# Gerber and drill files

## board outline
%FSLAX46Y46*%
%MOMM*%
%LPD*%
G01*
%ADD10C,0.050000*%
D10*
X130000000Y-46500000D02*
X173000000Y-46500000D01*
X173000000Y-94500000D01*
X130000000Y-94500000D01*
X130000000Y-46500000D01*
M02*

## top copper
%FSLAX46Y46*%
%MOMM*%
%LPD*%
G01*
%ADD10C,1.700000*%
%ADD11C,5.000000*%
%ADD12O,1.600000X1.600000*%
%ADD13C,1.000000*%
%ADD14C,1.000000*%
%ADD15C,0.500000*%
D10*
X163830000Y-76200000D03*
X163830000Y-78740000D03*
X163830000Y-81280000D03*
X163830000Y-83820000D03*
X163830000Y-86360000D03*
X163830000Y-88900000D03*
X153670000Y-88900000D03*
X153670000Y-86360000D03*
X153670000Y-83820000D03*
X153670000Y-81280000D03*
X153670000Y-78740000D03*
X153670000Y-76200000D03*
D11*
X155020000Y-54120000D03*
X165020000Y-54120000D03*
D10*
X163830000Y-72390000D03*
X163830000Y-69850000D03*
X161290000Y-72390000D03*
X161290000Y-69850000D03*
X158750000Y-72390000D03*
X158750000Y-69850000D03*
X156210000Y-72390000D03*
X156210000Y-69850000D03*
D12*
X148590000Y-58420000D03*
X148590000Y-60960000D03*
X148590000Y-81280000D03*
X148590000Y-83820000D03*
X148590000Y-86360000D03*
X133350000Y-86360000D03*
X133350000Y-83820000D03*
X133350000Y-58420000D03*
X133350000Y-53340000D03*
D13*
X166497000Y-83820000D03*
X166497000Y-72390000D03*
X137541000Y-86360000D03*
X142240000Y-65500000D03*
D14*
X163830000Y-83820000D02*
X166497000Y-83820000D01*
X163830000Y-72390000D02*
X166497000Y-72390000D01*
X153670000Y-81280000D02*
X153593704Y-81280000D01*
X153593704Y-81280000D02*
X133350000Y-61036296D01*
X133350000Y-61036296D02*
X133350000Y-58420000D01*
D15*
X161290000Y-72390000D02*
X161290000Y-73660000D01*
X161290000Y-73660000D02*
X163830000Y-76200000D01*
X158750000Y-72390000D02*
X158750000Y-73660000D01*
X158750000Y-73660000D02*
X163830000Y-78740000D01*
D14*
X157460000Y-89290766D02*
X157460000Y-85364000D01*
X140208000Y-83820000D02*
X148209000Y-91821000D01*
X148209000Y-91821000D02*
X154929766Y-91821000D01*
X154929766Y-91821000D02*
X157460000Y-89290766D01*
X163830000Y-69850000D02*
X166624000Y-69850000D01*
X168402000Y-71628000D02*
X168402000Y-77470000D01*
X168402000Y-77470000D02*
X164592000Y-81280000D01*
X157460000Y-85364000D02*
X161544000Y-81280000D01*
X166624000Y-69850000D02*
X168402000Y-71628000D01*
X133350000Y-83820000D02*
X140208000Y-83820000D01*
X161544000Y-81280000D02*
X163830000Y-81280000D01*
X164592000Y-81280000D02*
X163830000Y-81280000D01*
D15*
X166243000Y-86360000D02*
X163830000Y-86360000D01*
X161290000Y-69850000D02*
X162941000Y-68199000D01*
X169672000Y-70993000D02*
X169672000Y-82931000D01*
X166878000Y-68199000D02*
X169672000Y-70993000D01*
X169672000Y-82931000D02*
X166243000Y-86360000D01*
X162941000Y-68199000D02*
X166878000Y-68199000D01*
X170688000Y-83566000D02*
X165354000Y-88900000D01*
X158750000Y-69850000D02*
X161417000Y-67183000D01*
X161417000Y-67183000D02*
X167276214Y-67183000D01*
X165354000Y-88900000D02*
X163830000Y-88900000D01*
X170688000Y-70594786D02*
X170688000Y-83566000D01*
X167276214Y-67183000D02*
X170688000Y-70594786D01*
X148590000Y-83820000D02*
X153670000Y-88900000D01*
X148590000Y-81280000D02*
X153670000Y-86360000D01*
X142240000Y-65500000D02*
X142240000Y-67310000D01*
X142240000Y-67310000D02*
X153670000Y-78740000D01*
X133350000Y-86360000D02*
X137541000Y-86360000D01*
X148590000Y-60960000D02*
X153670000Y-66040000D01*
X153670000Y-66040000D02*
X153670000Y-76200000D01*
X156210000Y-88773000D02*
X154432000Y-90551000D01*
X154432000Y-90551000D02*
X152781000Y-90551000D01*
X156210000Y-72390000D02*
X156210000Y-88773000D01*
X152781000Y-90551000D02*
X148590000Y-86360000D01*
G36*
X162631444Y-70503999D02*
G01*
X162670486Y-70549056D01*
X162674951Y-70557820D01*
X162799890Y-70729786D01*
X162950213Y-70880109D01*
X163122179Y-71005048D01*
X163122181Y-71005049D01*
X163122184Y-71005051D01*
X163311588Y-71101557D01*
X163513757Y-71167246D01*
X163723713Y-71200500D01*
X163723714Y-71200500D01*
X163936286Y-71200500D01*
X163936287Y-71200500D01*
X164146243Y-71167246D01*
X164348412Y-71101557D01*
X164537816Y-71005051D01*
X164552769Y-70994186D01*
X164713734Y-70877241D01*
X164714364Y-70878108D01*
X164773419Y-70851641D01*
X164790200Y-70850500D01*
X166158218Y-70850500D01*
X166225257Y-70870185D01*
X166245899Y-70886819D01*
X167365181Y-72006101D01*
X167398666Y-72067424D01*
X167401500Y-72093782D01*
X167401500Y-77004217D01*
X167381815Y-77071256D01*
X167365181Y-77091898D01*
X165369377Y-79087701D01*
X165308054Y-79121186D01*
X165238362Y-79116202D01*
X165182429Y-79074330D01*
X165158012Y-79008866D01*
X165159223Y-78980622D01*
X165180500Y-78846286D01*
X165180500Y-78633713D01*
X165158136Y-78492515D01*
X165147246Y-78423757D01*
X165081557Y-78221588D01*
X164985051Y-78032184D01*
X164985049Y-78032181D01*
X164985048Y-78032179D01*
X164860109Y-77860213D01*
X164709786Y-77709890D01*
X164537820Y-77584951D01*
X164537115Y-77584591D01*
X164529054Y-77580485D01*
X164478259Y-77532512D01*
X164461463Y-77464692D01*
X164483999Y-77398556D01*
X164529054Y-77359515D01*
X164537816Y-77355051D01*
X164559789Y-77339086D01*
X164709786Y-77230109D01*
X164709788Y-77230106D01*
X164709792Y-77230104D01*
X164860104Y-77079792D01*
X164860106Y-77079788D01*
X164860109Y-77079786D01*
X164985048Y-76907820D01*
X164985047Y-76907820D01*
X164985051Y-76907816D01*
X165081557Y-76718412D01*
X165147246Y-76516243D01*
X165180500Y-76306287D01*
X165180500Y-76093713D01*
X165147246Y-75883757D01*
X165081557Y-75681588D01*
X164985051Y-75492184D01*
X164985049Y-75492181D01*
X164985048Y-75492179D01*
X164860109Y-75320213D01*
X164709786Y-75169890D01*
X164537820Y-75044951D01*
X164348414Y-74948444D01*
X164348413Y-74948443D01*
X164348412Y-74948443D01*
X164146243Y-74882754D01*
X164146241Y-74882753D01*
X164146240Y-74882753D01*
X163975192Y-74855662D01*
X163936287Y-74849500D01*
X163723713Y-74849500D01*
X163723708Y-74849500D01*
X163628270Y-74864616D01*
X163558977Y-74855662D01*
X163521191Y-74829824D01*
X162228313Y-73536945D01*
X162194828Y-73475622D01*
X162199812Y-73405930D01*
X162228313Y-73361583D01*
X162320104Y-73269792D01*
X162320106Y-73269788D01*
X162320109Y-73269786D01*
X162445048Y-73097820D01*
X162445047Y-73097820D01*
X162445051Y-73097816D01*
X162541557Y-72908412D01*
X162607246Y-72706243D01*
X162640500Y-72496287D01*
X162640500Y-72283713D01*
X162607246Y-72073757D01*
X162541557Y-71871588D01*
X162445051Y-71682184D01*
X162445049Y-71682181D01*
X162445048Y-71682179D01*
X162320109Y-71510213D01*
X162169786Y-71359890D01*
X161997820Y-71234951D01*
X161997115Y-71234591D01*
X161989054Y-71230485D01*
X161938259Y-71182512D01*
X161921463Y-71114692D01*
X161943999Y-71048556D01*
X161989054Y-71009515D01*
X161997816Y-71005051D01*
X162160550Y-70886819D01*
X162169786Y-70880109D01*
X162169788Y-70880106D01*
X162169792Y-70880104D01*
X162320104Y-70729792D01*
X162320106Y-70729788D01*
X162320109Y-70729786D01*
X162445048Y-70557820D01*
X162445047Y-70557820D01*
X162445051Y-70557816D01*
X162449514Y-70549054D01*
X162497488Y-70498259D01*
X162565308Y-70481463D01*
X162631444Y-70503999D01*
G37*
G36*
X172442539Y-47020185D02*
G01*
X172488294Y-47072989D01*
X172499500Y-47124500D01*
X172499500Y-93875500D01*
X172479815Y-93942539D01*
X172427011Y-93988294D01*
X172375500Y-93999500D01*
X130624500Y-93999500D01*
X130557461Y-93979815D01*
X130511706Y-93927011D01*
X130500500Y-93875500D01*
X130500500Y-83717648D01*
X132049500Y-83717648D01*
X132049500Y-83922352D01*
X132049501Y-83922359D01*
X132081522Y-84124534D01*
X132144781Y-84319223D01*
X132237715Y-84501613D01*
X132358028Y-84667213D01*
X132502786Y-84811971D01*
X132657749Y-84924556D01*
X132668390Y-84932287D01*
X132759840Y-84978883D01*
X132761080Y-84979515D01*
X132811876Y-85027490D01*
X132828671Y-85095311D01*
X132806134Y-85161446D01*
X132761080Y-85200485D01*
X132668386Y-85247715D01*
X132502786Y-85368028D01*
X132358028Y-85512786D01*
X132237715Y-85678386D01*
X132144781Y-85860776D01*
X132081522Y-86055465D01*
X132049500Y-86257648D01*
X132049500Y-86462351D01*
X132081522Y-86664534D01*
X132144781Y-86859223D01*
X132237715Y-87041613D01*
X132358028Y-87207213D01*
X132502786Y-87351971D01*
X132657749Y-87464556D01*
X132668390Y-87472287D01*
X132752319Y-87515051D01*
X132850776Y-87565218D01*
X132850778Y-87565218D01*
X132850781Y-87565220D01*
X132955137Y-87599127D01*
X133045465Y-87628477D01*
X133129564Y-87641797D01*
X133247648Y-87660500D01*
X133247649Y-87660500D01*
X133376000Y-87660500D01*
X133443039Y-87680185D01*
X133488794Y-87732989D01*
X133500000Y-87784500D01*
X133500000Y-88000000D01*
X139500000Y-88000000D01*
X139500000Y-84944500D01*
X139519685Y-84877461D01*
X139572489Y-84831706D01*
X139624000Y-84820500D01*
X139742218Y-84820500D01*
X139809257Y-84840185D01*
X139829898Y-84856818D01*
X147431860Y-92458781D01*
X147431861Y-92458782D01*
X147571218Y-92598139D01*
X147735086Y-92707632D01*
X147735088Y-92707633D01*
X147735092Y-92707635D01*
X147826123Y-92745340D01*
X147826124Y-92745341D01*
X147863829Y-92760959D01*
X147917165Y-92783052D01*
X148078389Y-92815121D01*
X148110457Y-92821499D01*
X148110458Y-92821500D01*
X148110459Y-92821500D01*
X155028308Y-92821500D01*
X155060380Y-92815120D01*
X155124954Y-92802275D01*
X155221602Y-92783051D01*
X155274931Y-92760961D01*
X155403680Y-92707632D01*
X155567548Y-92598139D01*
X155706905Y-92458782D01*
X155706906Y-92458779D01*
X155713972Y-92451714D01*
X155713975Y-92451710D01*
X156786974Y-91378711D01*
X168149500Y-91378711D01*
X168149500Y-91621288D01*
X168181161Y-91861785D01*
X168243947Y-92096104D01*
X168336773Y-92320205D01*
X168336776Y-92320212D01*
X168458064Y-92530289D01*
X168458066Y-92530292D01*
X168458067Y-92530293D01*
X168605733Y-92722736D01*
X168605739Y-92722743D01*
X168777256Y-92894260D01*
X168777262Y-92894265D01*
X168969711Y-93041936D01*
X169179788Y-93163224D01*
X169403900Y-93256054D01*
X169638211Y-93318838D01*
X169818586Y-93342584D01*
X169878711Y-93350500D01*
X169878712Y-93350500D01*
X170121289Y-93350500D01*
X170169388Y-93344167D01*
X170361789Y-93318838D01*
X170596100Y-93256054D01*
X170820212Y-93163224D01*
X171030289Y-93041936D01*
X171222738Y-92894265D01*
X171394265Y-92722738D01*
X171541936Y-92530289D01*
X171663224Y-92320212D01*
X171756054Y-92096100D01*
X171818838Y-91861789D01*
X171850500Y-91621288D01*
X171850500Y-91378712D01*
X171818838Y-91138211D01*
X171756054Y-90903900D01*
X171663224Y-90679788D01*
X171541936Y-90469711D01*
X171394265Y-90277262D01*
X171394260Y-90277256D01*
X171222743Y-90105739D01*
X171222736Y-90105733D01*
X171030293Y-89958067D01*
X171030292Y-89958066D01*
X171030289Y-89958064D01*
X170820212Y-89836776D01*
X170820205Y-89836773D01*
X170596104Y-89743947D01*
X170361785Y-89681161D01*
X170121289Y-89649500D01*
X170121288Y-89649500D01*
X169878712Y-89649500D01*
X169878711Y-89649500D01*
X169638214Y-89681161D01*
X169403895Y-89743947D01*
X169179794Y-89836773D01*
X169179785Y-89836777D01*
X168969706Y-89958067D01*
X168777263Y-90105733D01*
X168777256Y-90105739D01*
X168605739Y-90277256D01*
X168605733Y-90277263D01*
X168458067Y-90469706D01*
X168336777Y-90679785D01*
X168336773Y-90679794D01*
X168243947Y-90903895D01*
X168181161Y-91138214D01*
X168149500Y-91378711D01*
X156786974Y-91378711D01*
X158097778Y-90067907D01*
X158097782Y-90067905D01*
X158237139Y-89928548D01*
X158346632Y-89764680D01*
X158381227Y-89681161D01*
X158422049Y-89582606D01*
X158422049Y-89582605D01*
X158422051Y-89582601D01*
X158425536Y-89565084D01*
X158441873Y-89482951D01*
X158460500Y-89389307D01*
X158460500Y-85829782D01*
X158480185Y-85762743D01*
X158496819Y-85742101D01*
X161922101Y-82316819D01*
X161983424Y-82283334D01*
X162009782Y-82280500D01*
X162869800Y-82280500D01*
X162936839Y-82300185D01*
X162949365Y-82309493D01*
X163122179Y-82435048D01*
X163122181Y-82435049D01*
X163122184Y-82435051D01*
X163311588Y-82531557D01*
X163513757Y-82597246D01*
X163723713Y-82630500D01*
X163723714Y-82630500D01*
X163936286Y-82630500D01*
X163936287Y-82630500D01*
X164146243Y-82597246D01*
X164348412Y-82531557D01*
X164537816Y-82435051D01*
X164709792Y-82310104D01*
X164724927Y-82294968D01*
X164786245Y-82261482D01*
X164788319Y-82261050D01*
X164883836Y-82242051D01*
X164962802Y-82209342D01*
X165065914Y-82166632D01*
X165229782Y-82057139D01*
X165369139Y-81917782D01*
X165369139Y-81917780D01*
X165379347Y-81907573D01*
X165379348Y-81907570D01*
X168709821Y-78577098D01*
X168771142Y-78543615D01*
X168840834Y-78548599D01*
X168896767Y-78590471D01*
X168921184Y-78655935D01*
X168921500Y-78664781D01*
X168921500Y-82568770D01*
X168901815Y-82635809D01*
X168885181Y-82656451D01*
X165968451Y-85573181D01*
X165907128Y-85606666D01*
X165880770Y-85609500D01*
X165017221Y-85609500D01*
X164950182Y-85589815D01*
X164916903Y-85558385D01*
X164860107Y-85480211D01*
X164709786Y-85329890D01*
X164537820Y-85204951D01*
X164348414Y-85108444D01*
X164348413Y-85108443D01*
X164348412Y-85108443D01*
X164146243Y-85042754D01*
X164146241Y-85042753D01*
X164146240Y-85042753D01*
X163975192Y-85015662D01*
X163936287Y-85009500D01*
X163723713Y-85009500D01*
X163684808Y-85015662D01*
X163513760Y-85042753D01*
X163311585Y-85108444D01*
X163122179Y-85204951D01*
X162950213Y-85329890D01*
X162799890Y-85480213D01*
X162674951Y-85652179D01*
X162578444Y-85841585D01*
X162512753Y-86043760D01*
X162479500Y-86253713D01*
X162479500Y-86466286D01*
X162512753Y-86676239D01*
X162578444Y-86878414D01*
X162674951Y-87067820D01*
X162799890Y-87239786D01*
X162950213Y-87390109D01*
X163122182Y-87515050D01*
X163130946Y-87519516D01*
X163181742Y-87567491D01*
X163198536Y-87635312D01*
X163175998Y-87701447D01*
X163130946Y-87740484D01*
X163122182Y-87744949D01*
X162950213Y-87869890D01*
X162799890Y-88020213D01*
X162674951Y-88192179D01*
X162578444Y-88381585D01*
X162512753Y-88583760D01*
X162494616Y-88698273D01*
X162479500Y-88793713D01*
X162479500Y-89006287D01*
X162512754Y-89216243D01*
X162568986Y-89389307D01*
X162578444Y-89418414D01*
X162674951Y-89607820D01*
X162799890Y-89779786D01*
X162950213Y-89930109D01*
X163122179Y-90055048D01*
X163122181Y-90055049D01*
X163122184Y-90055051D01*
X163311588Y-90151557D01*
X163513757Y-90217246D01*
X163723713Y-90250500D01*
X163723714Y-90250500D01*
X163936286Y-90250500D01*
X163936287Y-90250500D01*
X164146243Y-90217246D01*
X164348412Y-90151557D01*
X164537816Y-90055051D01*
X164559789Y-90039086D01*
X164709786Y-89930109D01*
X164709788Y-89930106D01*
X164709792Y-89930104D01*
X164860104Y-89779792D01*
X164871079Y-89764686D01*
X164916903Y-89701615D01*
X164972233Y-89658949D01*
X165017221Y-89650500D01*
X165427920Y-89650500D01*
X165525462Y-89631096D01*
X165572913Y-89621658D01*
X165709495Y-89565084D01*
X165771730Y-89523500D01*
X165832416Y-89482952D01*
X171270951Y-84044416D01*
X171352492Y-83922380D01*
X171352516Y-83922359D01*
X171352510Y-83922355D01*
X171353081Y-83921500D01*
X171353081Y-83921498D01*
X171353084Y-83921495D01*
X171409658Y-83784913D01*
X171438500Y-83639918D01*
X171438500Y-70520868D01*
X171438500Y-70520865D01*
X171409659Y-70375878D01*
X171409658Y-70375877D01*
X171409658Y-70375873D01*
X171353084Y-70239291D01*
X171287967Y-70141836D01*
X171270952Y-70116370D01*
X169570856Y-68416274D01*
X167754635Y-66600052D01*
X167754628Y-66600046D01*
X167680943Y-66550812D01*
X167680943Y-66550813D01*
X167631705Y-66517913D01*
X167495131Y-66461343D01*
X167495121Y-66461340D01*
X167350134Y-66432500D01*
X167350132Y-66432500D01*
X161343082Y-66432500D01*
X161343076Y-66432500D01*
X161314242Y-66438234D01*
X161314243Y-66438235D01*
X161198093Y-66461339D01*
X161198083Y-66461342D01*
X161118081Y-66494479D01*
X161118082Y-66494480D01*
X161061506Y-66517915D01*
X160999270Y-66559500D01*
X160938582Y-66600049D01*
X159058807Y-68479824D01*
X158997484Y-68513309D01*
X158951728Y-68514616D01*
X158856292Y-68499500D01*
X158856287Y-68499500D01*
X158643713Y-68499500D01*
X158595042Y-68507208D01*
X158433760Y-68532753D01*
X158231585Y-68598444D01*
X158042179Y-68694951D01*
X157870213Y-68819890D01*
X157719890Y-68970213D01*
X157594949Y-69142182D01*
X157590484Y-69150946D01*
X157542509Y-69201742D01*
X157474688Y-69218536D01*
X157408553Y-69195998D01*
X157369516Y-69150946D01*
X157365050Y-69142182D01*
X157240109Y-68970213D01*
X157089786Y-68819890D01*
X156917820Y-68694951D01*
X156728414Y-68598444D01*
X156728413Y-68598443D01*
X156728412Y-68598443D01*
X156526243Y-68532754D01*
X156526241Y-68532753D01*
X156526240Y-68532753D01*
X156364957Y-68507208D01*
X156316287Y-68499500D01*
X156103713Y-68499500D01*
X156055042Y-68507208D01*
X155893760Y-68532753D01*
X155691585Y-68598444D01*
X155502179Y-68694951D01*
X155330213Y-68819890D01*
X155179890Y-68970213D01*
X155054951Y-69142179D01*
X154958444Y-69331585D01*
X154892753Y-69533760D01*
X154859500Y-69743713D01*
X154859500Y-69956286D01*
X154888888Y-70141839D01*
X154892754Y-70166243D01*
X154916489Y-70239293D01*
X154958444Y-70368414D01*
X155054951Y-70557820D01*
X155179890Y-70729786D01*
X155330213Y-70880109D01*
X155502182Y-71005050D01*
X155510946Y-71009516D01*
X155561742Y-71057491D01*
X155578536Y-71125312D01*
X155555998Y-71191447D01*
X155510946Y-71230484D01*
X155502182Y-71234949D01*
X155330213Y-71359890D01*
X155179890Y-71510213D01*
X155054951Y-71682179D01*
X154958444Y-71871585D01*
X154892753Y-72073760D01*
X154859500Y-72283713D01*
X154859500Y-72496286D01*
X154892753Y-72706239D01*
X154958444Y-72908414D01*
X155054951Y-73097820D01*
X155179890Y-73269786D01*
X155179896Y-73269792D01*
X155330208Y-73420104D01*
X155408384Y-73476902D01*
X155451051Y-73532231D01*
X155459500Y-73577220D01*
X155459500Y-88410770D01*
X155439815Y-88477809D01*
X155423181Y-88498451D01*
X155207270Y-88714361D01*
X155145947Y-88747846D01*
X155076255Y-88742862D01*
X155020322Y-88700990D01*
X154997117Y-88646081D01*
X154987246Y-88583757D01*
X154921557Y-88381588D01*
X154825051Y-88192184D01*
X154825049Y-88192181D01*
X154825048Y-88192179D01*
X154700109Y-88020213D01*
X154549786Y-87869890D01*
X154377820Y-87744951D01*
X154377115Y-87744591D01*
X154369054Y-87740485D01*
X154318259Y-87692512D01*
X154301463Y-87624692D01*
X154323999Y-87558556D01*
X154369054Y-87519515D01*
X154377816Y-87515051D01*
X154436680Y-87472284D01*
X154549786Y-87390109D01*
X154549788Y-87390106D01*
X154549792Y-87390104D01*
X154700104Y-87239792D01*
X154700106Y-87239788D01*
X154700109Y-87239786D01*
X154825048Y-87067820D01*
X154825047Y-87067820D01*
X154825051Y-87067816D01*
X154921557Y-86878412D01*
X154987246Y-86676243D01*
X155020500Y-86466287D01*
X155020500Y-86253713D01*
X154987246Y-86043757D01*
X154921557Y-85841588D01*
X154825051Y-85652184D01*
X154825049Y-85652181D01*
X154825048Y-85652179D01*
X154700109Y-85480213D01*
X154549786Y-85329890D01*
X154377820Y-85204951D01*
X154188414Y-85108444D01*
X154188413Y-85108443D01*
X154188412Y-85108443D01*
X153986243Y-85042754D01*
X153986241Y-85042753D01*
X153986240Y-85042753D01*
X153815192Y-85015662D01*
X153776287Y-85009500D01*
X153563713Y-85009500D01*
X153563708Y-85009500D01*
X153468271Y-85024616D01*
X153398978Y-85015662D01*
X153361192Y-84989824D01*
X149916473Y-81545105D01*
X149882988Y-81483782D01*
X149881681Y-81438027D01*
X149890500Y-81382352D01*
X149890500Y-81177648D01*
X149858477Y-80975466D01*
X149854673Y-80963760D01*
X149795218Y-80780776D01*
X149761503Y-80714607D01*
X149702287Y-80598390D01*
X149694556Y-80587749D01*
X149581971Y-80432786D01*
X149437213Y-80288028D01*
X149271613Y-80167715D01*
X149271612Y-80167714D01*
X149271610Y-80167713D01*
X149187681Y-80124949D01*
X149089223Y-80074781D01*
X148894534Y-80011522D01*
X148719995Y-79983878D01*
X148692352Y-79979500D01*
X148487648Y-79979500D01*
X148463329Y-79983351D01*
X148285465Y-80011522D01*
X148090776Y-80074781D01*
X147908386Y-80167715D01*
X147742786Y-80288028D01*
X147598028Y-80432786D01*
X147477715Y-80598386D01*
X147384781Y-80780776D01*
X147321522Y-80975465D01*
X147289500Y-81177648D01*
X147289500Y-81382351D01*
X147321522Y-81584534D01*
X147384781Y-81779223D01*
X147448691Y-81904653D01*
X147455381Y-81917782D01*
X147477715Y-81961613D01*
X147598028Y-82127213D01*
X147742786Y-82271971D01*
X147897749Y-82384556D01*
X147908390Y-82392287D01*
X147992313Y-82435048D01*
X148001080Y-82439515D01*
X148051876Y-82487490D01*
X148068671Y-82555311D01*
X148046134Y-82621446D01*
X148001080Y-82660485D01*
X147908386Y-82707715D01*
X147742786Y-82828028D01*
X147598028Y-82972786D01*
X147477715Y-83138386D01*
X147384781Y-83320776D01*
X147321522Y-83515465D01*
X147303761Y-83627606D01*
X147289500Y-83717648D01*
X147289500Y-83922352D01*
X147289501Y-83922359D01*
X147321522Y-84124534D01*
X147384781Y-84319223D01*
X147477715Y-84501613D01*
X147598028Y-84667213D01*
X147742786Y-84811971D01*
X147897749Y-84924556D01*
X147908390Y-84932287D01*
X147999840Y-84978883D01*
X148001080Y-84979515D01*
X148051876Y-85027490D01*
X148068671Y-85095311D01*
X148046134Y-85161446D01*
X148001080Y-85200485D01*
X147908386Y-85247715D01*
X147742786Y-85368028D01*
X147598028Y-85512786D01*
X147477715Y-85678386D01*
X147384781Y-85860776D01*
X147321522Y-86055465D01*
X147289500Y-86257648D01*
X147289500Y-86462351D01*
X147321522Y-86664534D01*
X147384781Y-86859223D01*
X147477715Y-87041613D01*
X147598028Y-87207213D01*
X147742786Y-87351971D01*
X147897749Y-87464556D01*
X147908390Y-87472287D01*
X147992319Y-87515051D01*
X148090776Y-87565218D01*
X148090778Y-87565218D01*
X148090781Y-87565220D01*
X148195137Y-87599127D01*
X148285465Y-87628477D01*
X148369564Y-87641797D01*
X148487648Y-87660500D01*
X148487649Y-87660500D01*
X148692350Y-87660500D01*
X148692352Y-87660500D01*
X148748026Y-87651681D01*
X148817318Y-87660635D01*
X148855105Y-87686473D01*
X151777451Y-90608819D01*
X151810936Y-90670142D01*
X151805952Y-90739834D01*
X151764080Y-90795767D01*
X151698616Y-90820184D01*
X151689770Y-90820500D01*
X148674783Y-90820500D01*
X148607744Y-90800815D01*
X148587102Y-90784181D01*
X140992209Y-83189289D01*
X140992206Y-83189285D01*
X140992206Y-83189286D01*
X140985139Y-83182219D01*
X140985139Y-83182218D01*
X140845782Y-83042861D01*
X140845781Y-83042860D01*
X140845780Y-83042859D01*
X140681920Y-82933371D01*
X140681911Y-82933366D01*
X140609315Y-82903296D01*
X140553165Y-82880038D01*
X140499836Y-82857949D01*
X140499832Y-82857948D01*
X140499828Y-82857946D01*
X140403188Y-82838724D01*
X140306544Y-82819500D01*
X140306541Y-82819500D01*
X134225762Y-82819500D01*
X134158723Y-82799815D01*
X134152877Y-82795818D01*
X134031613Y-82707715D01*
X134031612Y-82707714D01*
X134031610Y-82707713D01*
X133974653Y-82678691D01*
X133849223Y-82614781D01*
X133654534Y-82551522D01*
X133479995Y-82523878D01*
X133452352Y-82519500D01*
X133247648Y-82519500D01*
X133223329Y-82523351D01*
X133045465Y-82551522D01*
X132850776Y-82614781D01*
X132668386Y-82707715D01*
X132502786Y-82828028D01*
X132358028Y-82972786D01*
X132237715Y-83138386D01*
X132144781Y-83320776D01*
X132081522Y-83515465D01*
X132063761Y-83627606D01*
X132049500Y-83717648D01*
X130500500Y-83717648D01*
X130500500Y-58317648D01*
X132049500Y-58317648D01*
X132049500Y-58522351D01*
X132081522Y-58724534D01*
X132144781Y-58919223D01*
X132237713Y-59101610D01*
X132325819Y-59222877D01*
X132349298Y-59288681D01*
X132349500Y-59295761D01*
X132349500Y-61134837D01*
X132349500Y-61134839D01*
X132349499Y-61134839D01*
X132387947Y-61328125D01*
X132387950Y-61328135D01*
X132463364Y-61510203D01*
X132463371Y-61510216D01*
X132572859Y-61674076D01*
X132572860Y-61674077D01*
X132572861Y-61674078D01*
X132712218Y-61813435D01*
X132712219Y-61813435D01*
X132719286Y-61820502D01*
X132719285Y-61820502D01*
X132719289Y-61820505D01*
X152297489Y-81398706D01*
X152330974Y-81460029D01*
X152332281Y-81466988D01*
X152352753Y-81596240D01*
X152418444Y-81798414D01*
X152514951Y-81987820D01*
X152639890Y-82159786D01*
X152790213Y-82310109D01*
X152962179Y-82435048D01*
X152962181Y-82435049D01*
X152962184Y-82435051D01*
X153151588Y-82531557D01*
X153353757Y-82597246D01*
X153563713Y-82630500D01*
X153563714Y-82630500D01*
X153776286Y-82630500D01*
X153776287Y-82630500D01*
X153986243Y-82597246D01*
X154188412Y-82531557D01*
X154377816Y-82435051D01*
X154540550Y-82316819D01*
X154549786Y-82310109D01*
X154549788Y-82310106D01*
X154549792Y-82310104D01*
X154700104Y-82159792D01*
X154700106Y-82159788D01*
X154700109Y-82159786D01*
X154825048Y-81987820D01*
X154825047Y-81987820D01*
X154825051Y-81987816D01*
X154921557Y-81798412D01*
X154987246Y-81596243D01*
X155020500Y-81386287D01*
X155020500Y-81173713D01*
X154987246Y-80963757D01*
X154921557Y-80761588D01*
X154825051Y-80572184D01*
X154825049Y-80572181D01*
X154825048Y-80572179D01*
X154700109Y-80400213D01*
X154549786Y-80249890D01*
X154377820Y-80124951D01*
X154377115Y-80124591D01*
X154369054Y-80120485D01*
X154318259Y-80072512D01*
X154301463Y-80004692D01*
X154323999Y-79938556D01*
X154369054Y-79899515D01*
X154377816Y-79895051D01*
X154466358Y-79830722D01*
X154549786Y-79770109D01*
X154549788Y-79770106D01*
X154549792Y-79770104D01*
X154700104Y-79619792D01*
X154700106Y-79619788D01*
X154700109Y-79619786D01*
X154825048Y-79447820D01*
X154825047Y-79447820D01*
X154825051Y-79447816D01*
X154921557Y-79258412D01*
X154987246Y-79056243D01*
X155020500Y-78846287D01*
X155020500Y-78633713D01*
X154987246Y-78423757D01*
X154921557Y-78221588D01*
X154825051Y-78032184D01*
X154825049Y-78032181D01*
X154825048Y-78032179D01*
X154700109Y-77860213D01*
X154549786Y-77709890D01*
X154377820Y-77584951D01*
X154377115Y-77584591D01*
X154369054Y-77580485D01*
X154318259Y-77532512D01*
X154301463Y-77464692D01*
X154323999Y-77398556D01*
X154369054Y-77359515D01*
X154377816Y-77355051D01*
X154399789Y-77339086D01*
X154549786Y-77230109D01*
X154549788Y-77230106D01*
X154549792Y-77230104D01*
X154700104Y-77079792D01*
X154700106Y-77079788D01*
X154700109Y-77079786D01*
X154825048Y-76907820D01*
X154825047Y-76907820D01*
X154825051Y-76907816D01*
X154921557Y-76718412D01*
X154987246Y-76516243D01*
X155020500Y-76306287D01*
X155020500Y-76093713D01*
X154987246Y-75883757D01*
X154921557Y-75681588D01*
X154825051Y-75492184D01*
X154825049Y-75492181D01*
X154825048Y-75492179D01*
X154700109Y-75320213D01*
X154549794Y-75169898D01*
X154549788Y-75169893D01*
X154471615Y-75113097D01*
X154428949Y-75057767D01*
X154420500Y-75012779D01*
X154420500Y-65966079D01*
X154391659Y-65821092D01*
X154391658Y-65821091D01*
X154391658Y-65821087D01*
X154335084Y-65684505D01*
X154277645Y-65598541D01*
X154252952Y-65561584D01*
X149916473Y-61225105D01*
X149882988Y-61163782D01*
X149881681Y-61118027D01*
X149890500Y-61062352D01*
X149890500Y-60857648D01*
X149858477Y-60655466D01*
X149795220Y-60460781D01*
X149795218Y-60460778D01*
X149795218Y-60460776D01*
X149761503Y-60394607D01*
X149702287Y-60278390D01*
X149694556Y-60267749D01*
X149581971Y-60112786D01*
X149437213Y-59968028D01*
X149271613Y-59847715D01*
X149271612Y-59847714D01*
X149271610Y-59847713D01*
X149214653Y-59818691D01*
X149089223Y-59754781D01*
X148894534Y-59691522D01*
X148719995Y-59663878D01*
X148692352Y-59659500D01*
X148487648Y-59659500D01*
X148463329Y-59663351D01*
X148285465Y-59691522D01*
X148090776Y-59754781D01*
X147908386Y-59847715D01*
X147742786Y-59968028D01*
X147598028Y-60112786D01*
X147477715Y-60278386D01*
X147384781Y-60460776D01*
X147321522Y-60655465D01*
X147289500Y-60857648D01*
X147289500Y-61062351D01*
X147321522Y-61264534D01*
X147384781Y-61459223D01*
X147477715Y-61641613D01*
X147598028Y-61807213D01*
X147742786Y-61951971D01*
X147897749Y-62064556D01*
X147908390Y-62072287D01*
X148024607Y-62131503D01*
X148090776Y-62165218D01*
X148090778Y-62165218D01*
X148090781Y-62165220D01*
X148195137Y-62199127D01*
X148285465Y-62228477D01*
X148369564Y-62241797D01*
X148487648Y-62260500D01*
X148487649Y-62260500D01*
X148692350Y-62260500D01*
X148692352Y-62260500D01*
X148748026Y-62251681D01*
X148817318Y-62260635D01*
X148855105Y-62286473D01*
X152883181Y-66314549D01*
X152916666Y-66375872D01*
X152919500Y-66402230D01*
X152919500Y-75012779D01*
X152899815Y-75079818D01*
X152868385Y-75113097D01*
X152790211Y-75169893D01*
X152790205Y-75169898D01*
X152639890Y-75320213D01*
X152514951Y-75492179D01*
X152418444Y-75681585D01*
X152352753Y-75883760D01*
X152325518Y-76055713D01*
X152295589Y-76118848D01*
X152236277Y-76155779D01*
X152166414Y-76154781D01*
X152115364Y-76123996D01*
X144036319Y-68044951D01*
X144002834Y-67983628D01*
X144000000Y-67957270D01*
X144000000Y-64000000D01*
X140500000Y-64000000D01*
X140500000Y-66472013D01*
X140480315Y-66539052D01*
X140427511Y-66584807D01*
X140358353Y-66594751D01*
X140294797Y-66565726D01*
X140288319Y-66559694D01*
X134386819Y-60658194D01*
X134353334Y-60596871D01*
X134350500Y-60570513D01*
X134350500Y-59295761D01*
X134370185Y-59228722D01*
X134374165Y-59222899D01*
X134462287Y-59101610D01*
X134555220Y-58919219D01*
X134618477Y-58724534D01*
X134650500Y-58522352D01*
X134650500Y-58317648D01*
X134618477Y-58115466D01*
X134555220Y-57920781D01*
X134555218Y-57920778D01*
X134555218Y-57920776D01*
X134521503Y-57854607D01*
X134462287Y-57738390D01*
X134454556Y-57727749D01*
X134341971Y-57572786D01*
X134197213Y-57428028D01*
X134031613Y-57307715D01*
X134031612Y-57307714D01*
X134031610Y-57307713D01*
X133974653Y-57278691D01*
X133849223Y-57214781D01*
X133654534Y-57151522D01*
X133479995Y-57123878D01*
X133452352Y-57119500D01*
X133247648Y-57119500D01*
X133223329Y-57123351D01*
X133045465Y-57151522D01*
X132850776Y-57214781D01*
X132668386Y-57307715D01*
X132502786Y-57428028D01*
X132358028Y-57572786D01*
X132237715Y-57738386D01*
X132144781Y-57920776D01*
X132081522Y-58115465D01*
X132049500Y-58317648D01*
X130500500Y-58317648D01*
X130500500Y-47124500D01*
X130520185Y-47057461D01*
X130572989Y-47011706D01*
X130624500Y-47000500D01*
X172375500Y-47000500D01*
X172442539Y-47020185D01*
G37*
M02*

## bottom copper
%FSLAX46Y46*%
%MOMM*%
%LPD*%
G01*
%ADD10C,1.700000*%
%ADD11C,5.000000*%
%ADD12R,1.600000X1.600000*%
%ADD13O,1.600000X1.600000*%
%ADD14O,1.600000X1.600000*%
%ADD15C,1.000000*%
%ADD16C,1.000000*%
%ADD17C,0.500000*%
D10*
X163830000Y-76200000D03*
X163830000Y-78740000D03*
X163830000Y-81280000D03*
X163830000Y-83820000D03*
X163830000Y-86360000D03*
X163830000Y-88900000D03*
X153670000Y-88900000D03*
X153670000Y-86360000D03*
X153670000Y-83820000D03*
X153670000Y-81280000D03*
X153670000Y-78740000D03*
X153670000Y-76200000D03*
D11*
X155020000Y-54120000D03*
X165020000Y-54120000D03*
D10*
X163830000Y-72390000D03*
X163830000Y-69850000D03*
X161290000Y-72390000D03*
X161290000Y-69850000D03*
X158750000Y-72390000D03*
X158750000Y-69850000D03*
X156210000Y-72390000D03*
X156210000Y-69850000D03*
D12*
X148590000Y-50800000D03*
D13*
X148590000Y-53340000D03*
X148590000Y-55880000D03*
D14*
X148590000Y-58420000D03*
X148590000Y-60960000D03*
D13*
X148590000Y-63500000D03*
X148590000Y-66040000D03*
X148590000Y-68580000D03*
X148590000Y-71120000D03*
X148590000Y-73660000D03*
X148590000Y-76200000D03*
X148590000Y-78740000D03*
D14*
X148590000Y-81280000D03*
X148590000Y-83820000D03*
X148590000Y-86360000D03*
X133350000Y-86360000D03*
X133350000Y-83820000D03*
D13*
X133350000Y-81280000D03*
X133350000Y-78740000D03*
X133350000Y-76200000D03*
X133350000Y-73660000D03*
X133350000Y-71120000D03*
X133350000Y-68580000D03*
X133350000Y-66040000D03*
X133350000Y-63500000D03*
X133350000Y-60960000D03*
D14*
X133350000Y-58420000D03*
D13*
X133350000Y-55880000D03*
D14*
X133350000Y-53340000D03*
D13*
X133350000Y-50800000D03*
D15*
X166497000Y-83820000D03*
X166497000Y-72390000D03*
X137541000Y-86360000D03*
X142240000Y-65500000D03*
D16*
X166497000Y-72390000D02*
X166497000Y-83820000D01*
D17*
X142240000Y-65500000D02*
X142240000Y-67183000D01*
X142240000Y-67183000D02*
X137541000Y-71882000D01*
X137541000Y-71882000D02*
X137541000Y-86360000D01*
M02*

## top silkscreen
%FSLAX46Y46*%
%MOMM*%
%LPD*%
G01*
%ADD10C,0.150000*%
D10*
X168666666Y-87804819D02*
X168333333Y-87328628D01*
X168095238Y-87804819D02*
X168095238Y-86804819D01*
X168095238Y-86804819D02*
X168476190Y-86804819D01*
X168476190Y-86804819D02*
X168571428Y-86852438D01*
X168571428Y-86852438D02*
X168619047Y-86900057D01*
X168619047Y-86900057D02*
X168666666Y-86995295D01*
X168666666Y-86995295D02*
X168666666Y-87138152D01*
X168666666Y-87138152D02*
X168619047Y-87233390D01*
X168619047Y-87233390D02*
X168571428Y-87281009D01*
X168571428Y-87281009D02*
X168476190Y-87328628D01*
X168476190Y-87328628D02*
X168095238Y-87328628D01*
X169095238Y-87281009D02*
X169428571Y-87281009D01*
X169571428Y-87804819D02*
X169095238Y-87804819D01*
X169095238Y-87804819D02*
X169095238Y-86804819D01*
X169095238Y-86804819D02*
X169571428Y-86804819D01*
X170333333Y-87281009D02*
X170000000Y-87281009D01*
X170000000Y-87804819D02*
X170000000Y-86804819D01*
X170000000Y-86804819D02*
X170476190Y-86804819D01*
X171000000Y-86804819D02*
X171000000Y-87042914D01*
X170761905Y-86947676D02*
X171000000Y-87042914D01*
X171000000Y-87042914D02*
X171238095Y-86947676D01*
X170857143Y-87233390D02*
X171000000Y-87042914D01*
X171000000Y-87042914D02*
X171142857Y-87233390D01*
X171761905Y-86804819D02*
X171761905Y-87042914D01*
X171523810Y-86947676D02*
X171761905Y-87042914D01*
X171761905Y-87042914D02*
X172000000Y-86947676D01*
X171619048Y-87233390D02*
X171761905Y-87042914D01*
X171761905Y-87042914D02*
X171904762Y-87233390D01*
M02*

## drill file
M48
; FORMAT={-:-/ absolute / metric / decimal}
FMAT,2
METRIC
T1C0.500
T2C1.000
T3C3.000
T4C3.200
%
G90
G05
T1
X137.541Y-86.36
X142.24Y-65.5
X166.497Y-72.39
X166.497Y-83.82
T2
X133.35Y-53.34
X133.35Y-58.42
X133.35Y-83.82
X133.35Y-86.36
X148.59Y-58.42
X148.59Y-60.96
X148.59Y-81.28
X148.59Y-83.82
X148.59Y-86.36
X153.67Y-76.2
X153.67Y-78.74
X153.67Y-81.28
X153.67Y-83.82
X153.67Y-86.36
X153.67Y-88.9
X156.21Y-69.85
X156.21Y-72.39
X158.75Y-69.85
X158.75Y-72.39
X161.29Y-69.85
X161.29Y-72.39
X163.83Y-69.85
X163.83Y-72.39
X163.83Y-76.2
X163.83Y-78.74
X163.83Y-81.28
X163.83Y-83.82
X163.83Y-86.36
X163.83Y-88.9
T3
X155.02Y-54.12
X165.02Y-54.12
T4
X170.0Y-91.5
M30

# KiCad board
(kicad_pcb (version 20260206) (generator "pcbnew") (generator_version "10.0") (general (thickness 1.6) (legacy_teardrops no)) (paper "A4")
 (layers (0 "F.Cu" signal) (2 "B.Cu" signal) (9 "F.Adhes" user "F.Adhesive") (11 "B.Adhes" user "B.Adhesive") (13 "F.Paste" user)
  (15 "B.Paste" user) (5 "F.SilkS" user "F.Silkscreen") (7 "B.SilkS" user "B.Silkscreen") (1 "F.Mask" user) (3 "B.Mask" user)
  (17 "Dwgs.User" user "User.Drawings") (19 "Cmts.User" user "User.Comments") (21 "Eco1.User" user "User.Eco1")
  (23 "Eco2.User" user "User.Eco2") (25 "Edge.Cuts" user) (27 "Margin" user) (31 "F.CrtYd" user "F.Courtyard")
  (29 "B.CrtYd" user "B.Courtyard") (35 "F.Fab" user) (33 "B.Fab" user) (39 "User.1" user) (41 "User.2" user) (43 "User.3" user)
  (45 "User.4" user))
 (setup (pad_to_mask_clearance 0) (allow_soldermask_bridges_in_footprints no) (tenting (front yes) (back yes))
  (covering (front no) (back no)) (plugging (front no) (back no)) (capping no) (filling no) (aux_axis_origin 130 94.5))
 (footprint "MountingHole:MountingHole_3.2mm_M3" (layer "F.Cu") (at 170 91.5)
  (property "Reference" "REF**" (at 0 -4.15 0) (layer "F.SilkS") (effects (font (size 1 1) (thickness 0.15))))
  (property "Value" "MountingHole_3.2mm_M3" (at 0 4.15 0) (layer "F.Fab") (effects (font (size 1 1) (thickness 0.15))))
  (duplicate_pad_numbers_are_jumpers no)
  (pad "" np_thru_hole circle (at 0 0) (size 3.2 3.2) (drill 3.2) (layers "*.Cu" "*.Mask")))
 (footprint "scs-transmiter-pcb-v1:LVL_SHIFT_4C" (layer "B.Cu") (at 158.75 76.2 180)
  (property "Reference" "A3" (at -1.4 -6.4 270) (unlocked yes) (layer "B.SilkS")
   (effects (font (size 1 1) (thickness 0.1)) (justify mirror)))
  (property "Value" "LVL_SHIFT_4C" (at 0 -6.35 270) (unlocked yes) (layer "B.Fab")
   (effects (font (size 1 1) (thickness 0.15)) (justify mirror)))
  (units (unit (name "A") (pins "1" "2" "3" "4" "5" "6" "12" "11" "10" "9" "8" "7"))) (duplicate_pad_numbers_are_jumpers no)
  (pad "1" thru_hole circle (at -5.08 0 180) (size 1.7 1.7) (drill 1) (layers "*.Cu" "*.Mask") (remove_unused_layers no) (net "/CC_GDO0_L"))
  (pad "2" thru_hole circle (at -5.08 -2.54 180) (size 1.7 1.7) (drill 1) (layers "*.Cu" "*.Mask") (remove_unused_layers no)
   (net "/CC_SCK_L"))
  (pad "3" thru_hole circle (at -5.08 -5.08 180) (size 1.7 1.7) (drill 1) (layers "*.Cu" "*.Mask") (remove_unused_layers no) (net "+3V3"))
  (pad "4" thru_hole circle (at -5.08 -7.62 180) (size 1.7 1.7) (drill 1) (layers "*.Cu" "*.Mask") (remove_unused_layers no) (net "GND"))
  (pad "5" thru_hole circle (at -5.08 -10.16 180) (size 1.7 1.7) (drill 1) (layers "*.Cu" "*.Mask") (remove_unused_layers no)
   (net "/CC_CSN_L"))
  (pad "6" thru_hole circle (at -5.08 -12.7 180) (size 1.7 1.7) (drill 1) (layers "*.Cu" "*.Mask") (remove_unused_layers no)
   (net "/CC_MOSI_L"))
  (pad "7" thru_hole circle (at 5.08 -12.7 180) (size 1.7 1.7) (drill 1) (layers "*.Cu" "*.Mask") (remove_unused_layers no)
   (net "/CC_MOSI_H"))
  (pad "8" thru_hole circle (at 5.08 -10.16 180) (size 1.7 1.7) (drill 1) (layers "*.Cu" "*.Mask") (remove_unused_layers no)
   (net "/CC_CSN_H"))
  (pad "9" thru_hole circle (at 5.08 -7.62 180) (size 1.7 1.7) (drill 1) (layers "*.Cu" "*.Mask") (remove_unused_layers no) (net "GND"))
  (pad "10" thru_hole circle (at 5.08 -5.08 180) (size 1.7 1.7) (drill 1) (layers "*.Cu" "*.Mask") (remove_unused_layers no) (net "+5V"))
  (pad "11" thru_hole circle (at 5.08 -2.54 180) (size 1.7 1.7) (drill 1) (layers "*.Cu" "*.Mask") (remove_unused_layers no)
   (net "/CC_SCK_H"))
  (pad "12" thru_hole circle (at 5.08 0 180) (size 1.7 1.7) (drill 1) (layers "*.Cu" "*.Mask") (remove_unused_layers no) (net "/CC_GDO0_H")))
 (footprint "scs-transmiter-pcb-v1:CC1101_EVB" (layer "B.Cu") (at 160.02 71.12 90)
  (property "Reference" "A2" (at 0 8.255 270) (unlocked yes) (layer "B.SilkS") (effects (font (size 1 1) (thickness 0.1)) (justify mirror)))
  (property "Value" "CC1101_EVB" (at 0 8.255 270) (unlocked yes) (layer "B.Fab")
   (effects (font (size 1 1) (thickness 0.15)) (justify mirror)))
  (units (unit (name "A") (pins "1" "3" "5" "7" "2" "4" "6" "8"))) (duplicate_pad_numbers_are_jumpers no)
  (pad "" thru_hole circle (at 17 -5 90) (size 5 5) (drill 3) (layers "*.Cu" "*.Mask") (remove_unused_layers no) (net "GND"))
  (pad "" thru_hole circle (at 17 5 90) (size 5 5) (drill 3) (layers "*.Cu" "*.Mask") (remove_unused_layers no) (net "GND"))
  (pad "1" thru_hole circle (at -1.27 3.81 90) (size 1.7 1.7) (drill 1) (layers "*.Cu" "*.Mask") (remove_unused_layers no) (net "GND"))
  (pad "2" thru_hole circle (at 1.27 3.81 90) (size 1.7 1.7) (drill 1) (layers "*.Cu" "*.Mask") (remove_unused_layers no) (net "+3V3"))
  (pad "3" thru_hole circle (at -1.27 1.27 90) (size 1.7 1.7) (drill 1) (layers "*.Cu" "*.Mask") (remove_unused_layers no)
   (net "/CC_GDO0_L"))
  (pad "4" thru_hole circle (at 1.27 1.27 90) (size 1.7 1.7) (drill 1) (layers "*.Cu" "*.Mask") (remove_unused_layers no) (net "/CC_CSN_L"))
  (pad "5" thru_hole circle (at -1.27 -1.27 90) (size 1.7 1.7) (drill 1) (layers "*.Cu" "*.Mask") (remove_unused_layers no)
   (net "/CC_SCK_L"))
  (pad "6" thru_hole circle (at 1.27 -1.27 90) (size 1.7 1.7) (drill 1) (layers "*.Cu" "*.Mask") (remove_unused_layers no)
   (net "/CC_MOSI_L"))
  (pad "7" thru_hole circle (at -1.27 -3.81 90) (size 1.7 1.7) (drill 1) (layers "*.Cu" "*.Mask") (remove_unused_layers no)
   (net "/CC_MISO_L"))
  (pad "8" thru_hole circle (at 1.27 -3.81 90) (size 1.7 1.7) (drill 1) (layers "*.Cu" "*.Mask") (remove_unused_layers no)
   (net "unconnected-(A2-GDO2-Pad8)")))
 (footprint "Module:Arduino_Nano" (layer "B.Cu") (at 148.59 50.8 180)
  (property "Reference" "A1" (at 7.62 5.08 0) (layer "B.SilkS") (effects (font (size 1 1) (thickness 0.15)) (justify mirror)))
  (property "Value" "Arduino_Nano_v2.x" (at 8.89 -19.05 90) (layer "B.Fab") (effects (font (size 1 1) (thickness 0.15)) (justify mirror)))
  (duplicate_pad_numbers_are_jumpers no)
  (pad "1" smd rect (at 0 0 180) (size 1.6 1.6) (layers "B.Cu" "B.Mask" "B.Paste") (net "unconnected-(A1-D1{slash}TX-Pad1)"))
  (pad "2" smd oval (at 0 -2.54 180) (size 1.6 1.6) (layers "B.Cu" "B.Mask" "B.Paste") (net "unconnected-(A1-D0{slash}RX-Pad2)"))
  (pad "3" smd oval (at 0 -5.08 180) (size 1.6 1.6) (layers "B.Cu" "B.Mask" "B.Paste") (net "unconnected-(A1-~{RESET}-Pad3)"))
  (pad "4" thru_hole oval (at 0 -7.62 180) (size 1.6 1.6) (drill 1) (layers "*.Cu" "*.Mask") (remove_unused_layers no) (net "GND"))
  (pad "5" thru_hole oval (at 0 -10.16 180) (size 1.6 1.6) (drill 1) (layers "*.Cu" "*.Mask") (remove_unused_layers no) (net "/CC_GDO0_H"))
  (pad "6" smd oval (at 0 -12.7 180) (size 1.6 1.6) (layers "B.Cu" "B.Mask" "B.Paste") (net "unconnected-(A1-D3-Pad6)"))
  (pad "7" smd oval (at 0 -15.24 180) (size 1.6 1.6) (layers "B.Cu" "B.Mask" "B.Paste") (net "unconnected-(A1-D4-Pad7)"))
  (pad "8" smd oval (at 0 -17.78 180) (size 1.6 1.6) (layers "B.Cu" "B.Mask" "B.Paste") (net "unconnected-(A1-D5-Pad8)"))
  (pad "9" smd oval (at 0 -20.32 180) (size 1.6 1.6) (layers "B.Cu" "B.Mask" "B.Paste") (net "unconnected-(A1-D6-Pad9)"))
  (pad "10" smd oval (at 0 -22.86 180) (size 1.6 1.6) (layers "B.Cu" "B.Mask" "B.Paste") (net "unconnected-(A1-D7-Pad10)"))
  (pad "11" smd oval (at 0 -25.4 180) (size 1.6 1.6) (layers "B.Cu" "B.Mask" "B.Paste") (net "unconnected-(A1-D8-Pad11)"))
  (pad "12" smd oval (at 0 -27.94 180) (size 1.6 1.6) (layers "B.Cu" "B.Mask" "B.Paste") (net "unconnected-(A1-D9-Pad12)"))
  (pad "13" thru_hole oval (at 0 -30.48 180) (size 1.6 1.6) (drill 1) (layers "*.Cu" "*.Mask") (remove_unused_layers no) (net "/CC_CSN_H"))
  (pad "14" thru_hole oval (at 0 -33.02 180) (size 1.6 1.6) (drill 1) (layers "*.Cu" "*.Mask") (remove_unused_layers no) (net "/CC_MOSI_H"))
  (pad "15" thru_hole oval (at 0 -35.56 180) (size 1.6 1.6) (drill 1) (layers "*.Cu" "*.Mask") (remove_unused_layers no) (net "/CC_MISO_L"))
  (pad "16" thru_hole oval (at 15.24 -35.56 180) (size 1.6 1.6) (drill 1) (layers "*.Cu" "*.Mask") (remove_unused_layers no)
   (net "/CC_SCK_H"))
  (pad "17" thru_hole oval (at 15.24 -33.02 180) (size 1.6 1.6) (drill 1) (layers "*.Cu" "*.Mask") (remove_unused_layers no) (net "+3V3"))
  (pad "18" smd oval (at 15.24 -30.48 180) (size 1.6 1.6) (layers "B.Cu" "B.Mask" "B.Paste") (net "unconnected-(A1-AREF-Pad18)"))
  (pad "19" smd oval (at 15.24 -27.94 180) (size 1.6 1.6) (layers "B.Cu" "B.Mask" "B.Paste") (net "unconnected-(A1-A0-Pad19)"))
  (pad "20" smd oval (at 15.24 -25.4 180) (size 1.6 1.6) (layers "B.Cu" "B.Mask" "B.Paste") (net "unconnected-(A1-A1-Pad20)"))
  (pad "21" smd oval (at 15.24 -22.86 180) (size 1.6 1.6) (layers "B.Cu" "B.Mask" "B.Paste") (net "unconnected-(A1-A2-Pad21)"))
  (pad "22" smd oval (at 15.24 -20.32 180) (size 1.6 1.6) (layers "B.Cu" "B.Mask" "B.Paste") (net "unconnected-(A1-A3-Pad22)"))
  (pad "23" smd oval (at 15.24 -17.78 180) (size 1.6 1.6) (layers "B.Cu" "B.Mask" "B.Paste") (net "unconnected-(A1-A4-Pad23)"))
  (pad "24" smd oval (at 15.24 -15.24 180) (size 1.6 1.6) (layers "B.Cu" "B.Mask" "B.Paste") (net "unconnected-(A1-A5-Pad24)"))
  (pad "25" smd oval (at 15.24 -12.7 180) (size 1.6 1.6) (layers "B.Cu" "B.Mask" "B.Paste") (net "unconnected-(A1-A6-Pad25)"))
  (pad "26" smd oval (at 15.24 -10.16 180) (size 1.6 1.6) (layers "B.Cu" "B.Mask" "B.Paste") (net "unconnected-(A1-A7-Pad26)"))
  (pad "27" thru_hole oval (at 15.24 -7.62 180) (size 1.6 1.6) (drill 1) (layers "*.Cu" "*.Mask") (remove_unused_layers no) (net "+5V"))
  (pad "28" smd oval (at 15.24 -5.08 180) (size 1.6 1.6) (layers "B.Cu" "B.Mask" "B.Paste") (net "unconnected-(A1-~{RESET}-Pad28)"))
  (pad "29" thru_hole oval (at 15.24 -2.54 180) (size 1.6 1.6) (drill 1) (layers "*.Cu" "*.Mask") (remove_unused_layers no) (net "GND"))
  (pad "30" smd oval (at 15.24 0 180) (size 1.6 1.6) (layers "B.Cu" "B.Mask" "B.Paste") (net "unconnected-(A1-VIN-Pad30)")))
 (gr_rect (start 130 46.5) (end 173 94.5) (stroke (width 0.05) (type default)) (fill no) (layer "Edge.Cuts"))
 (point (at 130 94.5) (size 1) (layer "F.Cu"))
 (segment (start 163.83 83.82) (end 166.497 83.82) (width 1) (layer "F.Cu") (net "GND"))
 (segment (start 163.83 72.39) (end 166.497 72.39) (width 1) (layer "F.Cu") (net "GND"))
 (via (at 166.497 83.82) (size 1) (drill 0.5) (layers "F.Cu" "B.Cu") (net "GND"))
 (via (at 166.497 72.39) (size 1) (drill 0.5) (layers "F.Cu" "B.Cu") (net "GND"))
 (segment (start 166.497 72.39) (end 166.497 83.82) (width 1) (layer "B.Cu") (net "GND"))
 (segment (start 153.67 81.28) (end 153.593704 81.28) (width 1) (layer "F.Cu") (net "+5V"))
 (segment (start 153.593704 81.28) (end 133.35 61.036296) (width 1) (layer "F.Cu") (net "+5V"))
 (segment (start 133.35 61.036296) (end 133.35 58.42) (width 1) (layer "F.Cu") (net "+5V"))
 (segment (start 161.29 72.39) (end 161.29 73.66) (width 0.5) (layer "F.Cu") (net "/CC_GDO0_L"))
 (segment (start 161.29 73.66) (end 163.83 76.2) (width 0.5) (layer "F.Cu") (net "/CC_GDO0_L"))
 (segment (start 158.75 72.39) (end 158.75 73.66) (width 0.5) (layer "F.Cu") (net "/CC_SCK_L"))
 (segment (start 158.75 73.66) (end 163.83 78.74) (width 0.5) (layer "F.Cu") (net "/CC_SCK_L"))
 (segment (start 157.46 89.290766) (end 157.46 85.364) (width 1) (layer "F.Cu") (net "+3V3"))
 (segment (start 140.208 83.82) (end 148.209 91.821) (width 1) (layer "F.Cu") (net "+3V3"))
 (segment (start 148.209 91.821) (end 154.929766 91.821) (width 1) (layer "F.Cu") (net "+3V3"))
 (segment (start 154.929766 91.821) (end 157.46 89.290766) (width 1) (layer "F.Cu") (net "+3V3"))
 (segment (start 163.83 69.85) (end 166.624 69.85) (width 1) (layer "F.Cu") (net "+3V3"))
 (segment (start 168.402 71.628) (end 168.402 77.47) (width 1) (layer "F.Cu") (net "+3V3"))
 (segment (start 168.402 77.47) (end 164.592 81.28) (width 1) (layer "F.Cu") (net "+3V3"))
 (segment (start 157.46 85.364) (end 161.544 81.28) (width 1) (layer "F.Cu") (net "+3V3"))
 (segment (start 166.624 69.85) (end 168.402 71.628) (width 1) (layer "F.Cu") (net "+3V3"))
 (segment (start 133.35 83.82) (end 140.208 83.82) (width 1) (layer "F.Cu") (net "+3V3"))
 (segment (start 161.544 81.28) (end 163.83 81.28) (width 1) (layer "F.Cu") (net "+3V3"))
 (segment (start 164.592 81.28) (end 163.83 81.28) (width 1) (layer "F.Cu") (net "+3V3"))
 (segment (start 166.243 86.36) (end 163.83 86.36) (width 0.5) (layer "F.Cu") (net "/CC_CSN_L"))
 (segment (start 161.29 69.85) (end 162.941 68.199) (width 0.5) (layer "F.Cu") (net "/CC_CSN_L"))
 (segment (start 169.672 70.993) (end 169.672 82.931) (width 0.5) (layer "F.Cu") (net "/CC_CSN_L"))
 (segment (start 166.878 68.199) (end 169.672 70.993) (width 0.5) (layer "F.Cu") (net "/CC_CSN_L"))
 (segment (start 169.672 82.931) (end 166.243 86.36) (width 0.5) (layer "F.Cu") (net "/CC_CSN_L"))
 (segment (start 162.941 68.199) (end 166.878 68.199) (width 0.5) (layer "F.Cu") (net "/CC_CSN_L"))
 (segment (start 170.688 83.566) (end 165.354 88.9) (width 0.5) (layer "F.Cu") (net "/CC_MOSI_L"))
 (segment (start 158.75 69.85) (end 161.417 67.183) (width 0.5) (layer "F.Cu") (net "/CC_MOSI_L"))
 (segment (start 161.417 67.183) (end 167.276214 67.183) (width 0.5) (layer "F.Cu") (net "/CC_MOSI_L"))
 (segment (start 165.354 88.9) (end 163.83 88.9) (width 0.5) (layer "F.Cu") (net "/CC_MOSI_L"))
 (segment (start 170.688 70.594786) (end 170.688 83.566) (width 0.5) (layer "F.Cu") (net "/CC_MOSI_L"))
 (segment (start 167.276214 67.183) (end 170.688 70.594786) (width 0.5) (layer "F.Cu") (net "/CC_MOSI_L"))
 (segment (start 148.59 83.82) (end 153.67 88.9) (width 0.5) (layer "F.Cu") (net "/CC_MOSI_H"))
 (segment (start 148.59 81.28) (end 153.67 86.36) (width 0.5) (layer "F.Cu") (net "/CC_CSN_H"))
 (segment (start 142.24 65.5) (end 142.24 67.31) (width 0.5) (layer "F.Cu") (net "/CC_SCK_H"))
 (segment (start 142.24 67.31) (end 153.67 78.74) (width 0.5) (layer "F.Cu") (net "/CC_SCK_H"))
 (segment (start 133.35 86.36) (end 137.541 86.36) (width 0.5) (layer "F.Cu") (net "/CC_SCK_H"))
 (via (at 137.541 86.36) (size 1) (drill 0.5) (layers "F.Cu" "B.Cu") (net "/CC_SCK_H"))
 (via (at 142.24 65.5) (size 1) (drill 0.5) (layers "F.Cu" "B.Cu") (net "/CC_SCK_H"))
 (segment (start 142.24 65.5) (end 142.24 67.183) (width 0.5) (layer "B.Cu") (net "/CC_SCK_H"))
 (segment (start 142.24 67.183) (end 137.541 71.882) (width 0.5) (layer "B.Cu") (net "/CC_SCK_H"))
 (segment (start 137.541 71.882) (end 137.541 86.36) (width 0.5) (layer "B.Cu") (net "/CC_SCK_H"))
 (segment (start 148.59 60.96) (end 153.67 66.04) (width 0.5) (layer "F.Cu") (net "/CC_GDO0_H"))
 (segment (start 153.67 66.04) (end 153.67 76.2) (width 0.5) (layer "F.Cu") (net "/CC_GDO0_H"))
 (segment (start 156.21 88.773) (end 154.432 90.551) (width 0.5) (layer "F.Cu") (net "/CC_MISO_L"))
 (segment (start 154.432 90.551) (end 152.781 90.551) (width 0.5) (layer "F.Cu") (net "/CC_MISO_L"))
 (segment (start 156.21 72.39) (end 156.21 88.773) (width 0.5) (layer "F.Cu") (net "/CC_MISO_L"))
 (segment (start 152.781 90.551) (end 148.59 86.36) (width 0.5) (layer "F.Cu") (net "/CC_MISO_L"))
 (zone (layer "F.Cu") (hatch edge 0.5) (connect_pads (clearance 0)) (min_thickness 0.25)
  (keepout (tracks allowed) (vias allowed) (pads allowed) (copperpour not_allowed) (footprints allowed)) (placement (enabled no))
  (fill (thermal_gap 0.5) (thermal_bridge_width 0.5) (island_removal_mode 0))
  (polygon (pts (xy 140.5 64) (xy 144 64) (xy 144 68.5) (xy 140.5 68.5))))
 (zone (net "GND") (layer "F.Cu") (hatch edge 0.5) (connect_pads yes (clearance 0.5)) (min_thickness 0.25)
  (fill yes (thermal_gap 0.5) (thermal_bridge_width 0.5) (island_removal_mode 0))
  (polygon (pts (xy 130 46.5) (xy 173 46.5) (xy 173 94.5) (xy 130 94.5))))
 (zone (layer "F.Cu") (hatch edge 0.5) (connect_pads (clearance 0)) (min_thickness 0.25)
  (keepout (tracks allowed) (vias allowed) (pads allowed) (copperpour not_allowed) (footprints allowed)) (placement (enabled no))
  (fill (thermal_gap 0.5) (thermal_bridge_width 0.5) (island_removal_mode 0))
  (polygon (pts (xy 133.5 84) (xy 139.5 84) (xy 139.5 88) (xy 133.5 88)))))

